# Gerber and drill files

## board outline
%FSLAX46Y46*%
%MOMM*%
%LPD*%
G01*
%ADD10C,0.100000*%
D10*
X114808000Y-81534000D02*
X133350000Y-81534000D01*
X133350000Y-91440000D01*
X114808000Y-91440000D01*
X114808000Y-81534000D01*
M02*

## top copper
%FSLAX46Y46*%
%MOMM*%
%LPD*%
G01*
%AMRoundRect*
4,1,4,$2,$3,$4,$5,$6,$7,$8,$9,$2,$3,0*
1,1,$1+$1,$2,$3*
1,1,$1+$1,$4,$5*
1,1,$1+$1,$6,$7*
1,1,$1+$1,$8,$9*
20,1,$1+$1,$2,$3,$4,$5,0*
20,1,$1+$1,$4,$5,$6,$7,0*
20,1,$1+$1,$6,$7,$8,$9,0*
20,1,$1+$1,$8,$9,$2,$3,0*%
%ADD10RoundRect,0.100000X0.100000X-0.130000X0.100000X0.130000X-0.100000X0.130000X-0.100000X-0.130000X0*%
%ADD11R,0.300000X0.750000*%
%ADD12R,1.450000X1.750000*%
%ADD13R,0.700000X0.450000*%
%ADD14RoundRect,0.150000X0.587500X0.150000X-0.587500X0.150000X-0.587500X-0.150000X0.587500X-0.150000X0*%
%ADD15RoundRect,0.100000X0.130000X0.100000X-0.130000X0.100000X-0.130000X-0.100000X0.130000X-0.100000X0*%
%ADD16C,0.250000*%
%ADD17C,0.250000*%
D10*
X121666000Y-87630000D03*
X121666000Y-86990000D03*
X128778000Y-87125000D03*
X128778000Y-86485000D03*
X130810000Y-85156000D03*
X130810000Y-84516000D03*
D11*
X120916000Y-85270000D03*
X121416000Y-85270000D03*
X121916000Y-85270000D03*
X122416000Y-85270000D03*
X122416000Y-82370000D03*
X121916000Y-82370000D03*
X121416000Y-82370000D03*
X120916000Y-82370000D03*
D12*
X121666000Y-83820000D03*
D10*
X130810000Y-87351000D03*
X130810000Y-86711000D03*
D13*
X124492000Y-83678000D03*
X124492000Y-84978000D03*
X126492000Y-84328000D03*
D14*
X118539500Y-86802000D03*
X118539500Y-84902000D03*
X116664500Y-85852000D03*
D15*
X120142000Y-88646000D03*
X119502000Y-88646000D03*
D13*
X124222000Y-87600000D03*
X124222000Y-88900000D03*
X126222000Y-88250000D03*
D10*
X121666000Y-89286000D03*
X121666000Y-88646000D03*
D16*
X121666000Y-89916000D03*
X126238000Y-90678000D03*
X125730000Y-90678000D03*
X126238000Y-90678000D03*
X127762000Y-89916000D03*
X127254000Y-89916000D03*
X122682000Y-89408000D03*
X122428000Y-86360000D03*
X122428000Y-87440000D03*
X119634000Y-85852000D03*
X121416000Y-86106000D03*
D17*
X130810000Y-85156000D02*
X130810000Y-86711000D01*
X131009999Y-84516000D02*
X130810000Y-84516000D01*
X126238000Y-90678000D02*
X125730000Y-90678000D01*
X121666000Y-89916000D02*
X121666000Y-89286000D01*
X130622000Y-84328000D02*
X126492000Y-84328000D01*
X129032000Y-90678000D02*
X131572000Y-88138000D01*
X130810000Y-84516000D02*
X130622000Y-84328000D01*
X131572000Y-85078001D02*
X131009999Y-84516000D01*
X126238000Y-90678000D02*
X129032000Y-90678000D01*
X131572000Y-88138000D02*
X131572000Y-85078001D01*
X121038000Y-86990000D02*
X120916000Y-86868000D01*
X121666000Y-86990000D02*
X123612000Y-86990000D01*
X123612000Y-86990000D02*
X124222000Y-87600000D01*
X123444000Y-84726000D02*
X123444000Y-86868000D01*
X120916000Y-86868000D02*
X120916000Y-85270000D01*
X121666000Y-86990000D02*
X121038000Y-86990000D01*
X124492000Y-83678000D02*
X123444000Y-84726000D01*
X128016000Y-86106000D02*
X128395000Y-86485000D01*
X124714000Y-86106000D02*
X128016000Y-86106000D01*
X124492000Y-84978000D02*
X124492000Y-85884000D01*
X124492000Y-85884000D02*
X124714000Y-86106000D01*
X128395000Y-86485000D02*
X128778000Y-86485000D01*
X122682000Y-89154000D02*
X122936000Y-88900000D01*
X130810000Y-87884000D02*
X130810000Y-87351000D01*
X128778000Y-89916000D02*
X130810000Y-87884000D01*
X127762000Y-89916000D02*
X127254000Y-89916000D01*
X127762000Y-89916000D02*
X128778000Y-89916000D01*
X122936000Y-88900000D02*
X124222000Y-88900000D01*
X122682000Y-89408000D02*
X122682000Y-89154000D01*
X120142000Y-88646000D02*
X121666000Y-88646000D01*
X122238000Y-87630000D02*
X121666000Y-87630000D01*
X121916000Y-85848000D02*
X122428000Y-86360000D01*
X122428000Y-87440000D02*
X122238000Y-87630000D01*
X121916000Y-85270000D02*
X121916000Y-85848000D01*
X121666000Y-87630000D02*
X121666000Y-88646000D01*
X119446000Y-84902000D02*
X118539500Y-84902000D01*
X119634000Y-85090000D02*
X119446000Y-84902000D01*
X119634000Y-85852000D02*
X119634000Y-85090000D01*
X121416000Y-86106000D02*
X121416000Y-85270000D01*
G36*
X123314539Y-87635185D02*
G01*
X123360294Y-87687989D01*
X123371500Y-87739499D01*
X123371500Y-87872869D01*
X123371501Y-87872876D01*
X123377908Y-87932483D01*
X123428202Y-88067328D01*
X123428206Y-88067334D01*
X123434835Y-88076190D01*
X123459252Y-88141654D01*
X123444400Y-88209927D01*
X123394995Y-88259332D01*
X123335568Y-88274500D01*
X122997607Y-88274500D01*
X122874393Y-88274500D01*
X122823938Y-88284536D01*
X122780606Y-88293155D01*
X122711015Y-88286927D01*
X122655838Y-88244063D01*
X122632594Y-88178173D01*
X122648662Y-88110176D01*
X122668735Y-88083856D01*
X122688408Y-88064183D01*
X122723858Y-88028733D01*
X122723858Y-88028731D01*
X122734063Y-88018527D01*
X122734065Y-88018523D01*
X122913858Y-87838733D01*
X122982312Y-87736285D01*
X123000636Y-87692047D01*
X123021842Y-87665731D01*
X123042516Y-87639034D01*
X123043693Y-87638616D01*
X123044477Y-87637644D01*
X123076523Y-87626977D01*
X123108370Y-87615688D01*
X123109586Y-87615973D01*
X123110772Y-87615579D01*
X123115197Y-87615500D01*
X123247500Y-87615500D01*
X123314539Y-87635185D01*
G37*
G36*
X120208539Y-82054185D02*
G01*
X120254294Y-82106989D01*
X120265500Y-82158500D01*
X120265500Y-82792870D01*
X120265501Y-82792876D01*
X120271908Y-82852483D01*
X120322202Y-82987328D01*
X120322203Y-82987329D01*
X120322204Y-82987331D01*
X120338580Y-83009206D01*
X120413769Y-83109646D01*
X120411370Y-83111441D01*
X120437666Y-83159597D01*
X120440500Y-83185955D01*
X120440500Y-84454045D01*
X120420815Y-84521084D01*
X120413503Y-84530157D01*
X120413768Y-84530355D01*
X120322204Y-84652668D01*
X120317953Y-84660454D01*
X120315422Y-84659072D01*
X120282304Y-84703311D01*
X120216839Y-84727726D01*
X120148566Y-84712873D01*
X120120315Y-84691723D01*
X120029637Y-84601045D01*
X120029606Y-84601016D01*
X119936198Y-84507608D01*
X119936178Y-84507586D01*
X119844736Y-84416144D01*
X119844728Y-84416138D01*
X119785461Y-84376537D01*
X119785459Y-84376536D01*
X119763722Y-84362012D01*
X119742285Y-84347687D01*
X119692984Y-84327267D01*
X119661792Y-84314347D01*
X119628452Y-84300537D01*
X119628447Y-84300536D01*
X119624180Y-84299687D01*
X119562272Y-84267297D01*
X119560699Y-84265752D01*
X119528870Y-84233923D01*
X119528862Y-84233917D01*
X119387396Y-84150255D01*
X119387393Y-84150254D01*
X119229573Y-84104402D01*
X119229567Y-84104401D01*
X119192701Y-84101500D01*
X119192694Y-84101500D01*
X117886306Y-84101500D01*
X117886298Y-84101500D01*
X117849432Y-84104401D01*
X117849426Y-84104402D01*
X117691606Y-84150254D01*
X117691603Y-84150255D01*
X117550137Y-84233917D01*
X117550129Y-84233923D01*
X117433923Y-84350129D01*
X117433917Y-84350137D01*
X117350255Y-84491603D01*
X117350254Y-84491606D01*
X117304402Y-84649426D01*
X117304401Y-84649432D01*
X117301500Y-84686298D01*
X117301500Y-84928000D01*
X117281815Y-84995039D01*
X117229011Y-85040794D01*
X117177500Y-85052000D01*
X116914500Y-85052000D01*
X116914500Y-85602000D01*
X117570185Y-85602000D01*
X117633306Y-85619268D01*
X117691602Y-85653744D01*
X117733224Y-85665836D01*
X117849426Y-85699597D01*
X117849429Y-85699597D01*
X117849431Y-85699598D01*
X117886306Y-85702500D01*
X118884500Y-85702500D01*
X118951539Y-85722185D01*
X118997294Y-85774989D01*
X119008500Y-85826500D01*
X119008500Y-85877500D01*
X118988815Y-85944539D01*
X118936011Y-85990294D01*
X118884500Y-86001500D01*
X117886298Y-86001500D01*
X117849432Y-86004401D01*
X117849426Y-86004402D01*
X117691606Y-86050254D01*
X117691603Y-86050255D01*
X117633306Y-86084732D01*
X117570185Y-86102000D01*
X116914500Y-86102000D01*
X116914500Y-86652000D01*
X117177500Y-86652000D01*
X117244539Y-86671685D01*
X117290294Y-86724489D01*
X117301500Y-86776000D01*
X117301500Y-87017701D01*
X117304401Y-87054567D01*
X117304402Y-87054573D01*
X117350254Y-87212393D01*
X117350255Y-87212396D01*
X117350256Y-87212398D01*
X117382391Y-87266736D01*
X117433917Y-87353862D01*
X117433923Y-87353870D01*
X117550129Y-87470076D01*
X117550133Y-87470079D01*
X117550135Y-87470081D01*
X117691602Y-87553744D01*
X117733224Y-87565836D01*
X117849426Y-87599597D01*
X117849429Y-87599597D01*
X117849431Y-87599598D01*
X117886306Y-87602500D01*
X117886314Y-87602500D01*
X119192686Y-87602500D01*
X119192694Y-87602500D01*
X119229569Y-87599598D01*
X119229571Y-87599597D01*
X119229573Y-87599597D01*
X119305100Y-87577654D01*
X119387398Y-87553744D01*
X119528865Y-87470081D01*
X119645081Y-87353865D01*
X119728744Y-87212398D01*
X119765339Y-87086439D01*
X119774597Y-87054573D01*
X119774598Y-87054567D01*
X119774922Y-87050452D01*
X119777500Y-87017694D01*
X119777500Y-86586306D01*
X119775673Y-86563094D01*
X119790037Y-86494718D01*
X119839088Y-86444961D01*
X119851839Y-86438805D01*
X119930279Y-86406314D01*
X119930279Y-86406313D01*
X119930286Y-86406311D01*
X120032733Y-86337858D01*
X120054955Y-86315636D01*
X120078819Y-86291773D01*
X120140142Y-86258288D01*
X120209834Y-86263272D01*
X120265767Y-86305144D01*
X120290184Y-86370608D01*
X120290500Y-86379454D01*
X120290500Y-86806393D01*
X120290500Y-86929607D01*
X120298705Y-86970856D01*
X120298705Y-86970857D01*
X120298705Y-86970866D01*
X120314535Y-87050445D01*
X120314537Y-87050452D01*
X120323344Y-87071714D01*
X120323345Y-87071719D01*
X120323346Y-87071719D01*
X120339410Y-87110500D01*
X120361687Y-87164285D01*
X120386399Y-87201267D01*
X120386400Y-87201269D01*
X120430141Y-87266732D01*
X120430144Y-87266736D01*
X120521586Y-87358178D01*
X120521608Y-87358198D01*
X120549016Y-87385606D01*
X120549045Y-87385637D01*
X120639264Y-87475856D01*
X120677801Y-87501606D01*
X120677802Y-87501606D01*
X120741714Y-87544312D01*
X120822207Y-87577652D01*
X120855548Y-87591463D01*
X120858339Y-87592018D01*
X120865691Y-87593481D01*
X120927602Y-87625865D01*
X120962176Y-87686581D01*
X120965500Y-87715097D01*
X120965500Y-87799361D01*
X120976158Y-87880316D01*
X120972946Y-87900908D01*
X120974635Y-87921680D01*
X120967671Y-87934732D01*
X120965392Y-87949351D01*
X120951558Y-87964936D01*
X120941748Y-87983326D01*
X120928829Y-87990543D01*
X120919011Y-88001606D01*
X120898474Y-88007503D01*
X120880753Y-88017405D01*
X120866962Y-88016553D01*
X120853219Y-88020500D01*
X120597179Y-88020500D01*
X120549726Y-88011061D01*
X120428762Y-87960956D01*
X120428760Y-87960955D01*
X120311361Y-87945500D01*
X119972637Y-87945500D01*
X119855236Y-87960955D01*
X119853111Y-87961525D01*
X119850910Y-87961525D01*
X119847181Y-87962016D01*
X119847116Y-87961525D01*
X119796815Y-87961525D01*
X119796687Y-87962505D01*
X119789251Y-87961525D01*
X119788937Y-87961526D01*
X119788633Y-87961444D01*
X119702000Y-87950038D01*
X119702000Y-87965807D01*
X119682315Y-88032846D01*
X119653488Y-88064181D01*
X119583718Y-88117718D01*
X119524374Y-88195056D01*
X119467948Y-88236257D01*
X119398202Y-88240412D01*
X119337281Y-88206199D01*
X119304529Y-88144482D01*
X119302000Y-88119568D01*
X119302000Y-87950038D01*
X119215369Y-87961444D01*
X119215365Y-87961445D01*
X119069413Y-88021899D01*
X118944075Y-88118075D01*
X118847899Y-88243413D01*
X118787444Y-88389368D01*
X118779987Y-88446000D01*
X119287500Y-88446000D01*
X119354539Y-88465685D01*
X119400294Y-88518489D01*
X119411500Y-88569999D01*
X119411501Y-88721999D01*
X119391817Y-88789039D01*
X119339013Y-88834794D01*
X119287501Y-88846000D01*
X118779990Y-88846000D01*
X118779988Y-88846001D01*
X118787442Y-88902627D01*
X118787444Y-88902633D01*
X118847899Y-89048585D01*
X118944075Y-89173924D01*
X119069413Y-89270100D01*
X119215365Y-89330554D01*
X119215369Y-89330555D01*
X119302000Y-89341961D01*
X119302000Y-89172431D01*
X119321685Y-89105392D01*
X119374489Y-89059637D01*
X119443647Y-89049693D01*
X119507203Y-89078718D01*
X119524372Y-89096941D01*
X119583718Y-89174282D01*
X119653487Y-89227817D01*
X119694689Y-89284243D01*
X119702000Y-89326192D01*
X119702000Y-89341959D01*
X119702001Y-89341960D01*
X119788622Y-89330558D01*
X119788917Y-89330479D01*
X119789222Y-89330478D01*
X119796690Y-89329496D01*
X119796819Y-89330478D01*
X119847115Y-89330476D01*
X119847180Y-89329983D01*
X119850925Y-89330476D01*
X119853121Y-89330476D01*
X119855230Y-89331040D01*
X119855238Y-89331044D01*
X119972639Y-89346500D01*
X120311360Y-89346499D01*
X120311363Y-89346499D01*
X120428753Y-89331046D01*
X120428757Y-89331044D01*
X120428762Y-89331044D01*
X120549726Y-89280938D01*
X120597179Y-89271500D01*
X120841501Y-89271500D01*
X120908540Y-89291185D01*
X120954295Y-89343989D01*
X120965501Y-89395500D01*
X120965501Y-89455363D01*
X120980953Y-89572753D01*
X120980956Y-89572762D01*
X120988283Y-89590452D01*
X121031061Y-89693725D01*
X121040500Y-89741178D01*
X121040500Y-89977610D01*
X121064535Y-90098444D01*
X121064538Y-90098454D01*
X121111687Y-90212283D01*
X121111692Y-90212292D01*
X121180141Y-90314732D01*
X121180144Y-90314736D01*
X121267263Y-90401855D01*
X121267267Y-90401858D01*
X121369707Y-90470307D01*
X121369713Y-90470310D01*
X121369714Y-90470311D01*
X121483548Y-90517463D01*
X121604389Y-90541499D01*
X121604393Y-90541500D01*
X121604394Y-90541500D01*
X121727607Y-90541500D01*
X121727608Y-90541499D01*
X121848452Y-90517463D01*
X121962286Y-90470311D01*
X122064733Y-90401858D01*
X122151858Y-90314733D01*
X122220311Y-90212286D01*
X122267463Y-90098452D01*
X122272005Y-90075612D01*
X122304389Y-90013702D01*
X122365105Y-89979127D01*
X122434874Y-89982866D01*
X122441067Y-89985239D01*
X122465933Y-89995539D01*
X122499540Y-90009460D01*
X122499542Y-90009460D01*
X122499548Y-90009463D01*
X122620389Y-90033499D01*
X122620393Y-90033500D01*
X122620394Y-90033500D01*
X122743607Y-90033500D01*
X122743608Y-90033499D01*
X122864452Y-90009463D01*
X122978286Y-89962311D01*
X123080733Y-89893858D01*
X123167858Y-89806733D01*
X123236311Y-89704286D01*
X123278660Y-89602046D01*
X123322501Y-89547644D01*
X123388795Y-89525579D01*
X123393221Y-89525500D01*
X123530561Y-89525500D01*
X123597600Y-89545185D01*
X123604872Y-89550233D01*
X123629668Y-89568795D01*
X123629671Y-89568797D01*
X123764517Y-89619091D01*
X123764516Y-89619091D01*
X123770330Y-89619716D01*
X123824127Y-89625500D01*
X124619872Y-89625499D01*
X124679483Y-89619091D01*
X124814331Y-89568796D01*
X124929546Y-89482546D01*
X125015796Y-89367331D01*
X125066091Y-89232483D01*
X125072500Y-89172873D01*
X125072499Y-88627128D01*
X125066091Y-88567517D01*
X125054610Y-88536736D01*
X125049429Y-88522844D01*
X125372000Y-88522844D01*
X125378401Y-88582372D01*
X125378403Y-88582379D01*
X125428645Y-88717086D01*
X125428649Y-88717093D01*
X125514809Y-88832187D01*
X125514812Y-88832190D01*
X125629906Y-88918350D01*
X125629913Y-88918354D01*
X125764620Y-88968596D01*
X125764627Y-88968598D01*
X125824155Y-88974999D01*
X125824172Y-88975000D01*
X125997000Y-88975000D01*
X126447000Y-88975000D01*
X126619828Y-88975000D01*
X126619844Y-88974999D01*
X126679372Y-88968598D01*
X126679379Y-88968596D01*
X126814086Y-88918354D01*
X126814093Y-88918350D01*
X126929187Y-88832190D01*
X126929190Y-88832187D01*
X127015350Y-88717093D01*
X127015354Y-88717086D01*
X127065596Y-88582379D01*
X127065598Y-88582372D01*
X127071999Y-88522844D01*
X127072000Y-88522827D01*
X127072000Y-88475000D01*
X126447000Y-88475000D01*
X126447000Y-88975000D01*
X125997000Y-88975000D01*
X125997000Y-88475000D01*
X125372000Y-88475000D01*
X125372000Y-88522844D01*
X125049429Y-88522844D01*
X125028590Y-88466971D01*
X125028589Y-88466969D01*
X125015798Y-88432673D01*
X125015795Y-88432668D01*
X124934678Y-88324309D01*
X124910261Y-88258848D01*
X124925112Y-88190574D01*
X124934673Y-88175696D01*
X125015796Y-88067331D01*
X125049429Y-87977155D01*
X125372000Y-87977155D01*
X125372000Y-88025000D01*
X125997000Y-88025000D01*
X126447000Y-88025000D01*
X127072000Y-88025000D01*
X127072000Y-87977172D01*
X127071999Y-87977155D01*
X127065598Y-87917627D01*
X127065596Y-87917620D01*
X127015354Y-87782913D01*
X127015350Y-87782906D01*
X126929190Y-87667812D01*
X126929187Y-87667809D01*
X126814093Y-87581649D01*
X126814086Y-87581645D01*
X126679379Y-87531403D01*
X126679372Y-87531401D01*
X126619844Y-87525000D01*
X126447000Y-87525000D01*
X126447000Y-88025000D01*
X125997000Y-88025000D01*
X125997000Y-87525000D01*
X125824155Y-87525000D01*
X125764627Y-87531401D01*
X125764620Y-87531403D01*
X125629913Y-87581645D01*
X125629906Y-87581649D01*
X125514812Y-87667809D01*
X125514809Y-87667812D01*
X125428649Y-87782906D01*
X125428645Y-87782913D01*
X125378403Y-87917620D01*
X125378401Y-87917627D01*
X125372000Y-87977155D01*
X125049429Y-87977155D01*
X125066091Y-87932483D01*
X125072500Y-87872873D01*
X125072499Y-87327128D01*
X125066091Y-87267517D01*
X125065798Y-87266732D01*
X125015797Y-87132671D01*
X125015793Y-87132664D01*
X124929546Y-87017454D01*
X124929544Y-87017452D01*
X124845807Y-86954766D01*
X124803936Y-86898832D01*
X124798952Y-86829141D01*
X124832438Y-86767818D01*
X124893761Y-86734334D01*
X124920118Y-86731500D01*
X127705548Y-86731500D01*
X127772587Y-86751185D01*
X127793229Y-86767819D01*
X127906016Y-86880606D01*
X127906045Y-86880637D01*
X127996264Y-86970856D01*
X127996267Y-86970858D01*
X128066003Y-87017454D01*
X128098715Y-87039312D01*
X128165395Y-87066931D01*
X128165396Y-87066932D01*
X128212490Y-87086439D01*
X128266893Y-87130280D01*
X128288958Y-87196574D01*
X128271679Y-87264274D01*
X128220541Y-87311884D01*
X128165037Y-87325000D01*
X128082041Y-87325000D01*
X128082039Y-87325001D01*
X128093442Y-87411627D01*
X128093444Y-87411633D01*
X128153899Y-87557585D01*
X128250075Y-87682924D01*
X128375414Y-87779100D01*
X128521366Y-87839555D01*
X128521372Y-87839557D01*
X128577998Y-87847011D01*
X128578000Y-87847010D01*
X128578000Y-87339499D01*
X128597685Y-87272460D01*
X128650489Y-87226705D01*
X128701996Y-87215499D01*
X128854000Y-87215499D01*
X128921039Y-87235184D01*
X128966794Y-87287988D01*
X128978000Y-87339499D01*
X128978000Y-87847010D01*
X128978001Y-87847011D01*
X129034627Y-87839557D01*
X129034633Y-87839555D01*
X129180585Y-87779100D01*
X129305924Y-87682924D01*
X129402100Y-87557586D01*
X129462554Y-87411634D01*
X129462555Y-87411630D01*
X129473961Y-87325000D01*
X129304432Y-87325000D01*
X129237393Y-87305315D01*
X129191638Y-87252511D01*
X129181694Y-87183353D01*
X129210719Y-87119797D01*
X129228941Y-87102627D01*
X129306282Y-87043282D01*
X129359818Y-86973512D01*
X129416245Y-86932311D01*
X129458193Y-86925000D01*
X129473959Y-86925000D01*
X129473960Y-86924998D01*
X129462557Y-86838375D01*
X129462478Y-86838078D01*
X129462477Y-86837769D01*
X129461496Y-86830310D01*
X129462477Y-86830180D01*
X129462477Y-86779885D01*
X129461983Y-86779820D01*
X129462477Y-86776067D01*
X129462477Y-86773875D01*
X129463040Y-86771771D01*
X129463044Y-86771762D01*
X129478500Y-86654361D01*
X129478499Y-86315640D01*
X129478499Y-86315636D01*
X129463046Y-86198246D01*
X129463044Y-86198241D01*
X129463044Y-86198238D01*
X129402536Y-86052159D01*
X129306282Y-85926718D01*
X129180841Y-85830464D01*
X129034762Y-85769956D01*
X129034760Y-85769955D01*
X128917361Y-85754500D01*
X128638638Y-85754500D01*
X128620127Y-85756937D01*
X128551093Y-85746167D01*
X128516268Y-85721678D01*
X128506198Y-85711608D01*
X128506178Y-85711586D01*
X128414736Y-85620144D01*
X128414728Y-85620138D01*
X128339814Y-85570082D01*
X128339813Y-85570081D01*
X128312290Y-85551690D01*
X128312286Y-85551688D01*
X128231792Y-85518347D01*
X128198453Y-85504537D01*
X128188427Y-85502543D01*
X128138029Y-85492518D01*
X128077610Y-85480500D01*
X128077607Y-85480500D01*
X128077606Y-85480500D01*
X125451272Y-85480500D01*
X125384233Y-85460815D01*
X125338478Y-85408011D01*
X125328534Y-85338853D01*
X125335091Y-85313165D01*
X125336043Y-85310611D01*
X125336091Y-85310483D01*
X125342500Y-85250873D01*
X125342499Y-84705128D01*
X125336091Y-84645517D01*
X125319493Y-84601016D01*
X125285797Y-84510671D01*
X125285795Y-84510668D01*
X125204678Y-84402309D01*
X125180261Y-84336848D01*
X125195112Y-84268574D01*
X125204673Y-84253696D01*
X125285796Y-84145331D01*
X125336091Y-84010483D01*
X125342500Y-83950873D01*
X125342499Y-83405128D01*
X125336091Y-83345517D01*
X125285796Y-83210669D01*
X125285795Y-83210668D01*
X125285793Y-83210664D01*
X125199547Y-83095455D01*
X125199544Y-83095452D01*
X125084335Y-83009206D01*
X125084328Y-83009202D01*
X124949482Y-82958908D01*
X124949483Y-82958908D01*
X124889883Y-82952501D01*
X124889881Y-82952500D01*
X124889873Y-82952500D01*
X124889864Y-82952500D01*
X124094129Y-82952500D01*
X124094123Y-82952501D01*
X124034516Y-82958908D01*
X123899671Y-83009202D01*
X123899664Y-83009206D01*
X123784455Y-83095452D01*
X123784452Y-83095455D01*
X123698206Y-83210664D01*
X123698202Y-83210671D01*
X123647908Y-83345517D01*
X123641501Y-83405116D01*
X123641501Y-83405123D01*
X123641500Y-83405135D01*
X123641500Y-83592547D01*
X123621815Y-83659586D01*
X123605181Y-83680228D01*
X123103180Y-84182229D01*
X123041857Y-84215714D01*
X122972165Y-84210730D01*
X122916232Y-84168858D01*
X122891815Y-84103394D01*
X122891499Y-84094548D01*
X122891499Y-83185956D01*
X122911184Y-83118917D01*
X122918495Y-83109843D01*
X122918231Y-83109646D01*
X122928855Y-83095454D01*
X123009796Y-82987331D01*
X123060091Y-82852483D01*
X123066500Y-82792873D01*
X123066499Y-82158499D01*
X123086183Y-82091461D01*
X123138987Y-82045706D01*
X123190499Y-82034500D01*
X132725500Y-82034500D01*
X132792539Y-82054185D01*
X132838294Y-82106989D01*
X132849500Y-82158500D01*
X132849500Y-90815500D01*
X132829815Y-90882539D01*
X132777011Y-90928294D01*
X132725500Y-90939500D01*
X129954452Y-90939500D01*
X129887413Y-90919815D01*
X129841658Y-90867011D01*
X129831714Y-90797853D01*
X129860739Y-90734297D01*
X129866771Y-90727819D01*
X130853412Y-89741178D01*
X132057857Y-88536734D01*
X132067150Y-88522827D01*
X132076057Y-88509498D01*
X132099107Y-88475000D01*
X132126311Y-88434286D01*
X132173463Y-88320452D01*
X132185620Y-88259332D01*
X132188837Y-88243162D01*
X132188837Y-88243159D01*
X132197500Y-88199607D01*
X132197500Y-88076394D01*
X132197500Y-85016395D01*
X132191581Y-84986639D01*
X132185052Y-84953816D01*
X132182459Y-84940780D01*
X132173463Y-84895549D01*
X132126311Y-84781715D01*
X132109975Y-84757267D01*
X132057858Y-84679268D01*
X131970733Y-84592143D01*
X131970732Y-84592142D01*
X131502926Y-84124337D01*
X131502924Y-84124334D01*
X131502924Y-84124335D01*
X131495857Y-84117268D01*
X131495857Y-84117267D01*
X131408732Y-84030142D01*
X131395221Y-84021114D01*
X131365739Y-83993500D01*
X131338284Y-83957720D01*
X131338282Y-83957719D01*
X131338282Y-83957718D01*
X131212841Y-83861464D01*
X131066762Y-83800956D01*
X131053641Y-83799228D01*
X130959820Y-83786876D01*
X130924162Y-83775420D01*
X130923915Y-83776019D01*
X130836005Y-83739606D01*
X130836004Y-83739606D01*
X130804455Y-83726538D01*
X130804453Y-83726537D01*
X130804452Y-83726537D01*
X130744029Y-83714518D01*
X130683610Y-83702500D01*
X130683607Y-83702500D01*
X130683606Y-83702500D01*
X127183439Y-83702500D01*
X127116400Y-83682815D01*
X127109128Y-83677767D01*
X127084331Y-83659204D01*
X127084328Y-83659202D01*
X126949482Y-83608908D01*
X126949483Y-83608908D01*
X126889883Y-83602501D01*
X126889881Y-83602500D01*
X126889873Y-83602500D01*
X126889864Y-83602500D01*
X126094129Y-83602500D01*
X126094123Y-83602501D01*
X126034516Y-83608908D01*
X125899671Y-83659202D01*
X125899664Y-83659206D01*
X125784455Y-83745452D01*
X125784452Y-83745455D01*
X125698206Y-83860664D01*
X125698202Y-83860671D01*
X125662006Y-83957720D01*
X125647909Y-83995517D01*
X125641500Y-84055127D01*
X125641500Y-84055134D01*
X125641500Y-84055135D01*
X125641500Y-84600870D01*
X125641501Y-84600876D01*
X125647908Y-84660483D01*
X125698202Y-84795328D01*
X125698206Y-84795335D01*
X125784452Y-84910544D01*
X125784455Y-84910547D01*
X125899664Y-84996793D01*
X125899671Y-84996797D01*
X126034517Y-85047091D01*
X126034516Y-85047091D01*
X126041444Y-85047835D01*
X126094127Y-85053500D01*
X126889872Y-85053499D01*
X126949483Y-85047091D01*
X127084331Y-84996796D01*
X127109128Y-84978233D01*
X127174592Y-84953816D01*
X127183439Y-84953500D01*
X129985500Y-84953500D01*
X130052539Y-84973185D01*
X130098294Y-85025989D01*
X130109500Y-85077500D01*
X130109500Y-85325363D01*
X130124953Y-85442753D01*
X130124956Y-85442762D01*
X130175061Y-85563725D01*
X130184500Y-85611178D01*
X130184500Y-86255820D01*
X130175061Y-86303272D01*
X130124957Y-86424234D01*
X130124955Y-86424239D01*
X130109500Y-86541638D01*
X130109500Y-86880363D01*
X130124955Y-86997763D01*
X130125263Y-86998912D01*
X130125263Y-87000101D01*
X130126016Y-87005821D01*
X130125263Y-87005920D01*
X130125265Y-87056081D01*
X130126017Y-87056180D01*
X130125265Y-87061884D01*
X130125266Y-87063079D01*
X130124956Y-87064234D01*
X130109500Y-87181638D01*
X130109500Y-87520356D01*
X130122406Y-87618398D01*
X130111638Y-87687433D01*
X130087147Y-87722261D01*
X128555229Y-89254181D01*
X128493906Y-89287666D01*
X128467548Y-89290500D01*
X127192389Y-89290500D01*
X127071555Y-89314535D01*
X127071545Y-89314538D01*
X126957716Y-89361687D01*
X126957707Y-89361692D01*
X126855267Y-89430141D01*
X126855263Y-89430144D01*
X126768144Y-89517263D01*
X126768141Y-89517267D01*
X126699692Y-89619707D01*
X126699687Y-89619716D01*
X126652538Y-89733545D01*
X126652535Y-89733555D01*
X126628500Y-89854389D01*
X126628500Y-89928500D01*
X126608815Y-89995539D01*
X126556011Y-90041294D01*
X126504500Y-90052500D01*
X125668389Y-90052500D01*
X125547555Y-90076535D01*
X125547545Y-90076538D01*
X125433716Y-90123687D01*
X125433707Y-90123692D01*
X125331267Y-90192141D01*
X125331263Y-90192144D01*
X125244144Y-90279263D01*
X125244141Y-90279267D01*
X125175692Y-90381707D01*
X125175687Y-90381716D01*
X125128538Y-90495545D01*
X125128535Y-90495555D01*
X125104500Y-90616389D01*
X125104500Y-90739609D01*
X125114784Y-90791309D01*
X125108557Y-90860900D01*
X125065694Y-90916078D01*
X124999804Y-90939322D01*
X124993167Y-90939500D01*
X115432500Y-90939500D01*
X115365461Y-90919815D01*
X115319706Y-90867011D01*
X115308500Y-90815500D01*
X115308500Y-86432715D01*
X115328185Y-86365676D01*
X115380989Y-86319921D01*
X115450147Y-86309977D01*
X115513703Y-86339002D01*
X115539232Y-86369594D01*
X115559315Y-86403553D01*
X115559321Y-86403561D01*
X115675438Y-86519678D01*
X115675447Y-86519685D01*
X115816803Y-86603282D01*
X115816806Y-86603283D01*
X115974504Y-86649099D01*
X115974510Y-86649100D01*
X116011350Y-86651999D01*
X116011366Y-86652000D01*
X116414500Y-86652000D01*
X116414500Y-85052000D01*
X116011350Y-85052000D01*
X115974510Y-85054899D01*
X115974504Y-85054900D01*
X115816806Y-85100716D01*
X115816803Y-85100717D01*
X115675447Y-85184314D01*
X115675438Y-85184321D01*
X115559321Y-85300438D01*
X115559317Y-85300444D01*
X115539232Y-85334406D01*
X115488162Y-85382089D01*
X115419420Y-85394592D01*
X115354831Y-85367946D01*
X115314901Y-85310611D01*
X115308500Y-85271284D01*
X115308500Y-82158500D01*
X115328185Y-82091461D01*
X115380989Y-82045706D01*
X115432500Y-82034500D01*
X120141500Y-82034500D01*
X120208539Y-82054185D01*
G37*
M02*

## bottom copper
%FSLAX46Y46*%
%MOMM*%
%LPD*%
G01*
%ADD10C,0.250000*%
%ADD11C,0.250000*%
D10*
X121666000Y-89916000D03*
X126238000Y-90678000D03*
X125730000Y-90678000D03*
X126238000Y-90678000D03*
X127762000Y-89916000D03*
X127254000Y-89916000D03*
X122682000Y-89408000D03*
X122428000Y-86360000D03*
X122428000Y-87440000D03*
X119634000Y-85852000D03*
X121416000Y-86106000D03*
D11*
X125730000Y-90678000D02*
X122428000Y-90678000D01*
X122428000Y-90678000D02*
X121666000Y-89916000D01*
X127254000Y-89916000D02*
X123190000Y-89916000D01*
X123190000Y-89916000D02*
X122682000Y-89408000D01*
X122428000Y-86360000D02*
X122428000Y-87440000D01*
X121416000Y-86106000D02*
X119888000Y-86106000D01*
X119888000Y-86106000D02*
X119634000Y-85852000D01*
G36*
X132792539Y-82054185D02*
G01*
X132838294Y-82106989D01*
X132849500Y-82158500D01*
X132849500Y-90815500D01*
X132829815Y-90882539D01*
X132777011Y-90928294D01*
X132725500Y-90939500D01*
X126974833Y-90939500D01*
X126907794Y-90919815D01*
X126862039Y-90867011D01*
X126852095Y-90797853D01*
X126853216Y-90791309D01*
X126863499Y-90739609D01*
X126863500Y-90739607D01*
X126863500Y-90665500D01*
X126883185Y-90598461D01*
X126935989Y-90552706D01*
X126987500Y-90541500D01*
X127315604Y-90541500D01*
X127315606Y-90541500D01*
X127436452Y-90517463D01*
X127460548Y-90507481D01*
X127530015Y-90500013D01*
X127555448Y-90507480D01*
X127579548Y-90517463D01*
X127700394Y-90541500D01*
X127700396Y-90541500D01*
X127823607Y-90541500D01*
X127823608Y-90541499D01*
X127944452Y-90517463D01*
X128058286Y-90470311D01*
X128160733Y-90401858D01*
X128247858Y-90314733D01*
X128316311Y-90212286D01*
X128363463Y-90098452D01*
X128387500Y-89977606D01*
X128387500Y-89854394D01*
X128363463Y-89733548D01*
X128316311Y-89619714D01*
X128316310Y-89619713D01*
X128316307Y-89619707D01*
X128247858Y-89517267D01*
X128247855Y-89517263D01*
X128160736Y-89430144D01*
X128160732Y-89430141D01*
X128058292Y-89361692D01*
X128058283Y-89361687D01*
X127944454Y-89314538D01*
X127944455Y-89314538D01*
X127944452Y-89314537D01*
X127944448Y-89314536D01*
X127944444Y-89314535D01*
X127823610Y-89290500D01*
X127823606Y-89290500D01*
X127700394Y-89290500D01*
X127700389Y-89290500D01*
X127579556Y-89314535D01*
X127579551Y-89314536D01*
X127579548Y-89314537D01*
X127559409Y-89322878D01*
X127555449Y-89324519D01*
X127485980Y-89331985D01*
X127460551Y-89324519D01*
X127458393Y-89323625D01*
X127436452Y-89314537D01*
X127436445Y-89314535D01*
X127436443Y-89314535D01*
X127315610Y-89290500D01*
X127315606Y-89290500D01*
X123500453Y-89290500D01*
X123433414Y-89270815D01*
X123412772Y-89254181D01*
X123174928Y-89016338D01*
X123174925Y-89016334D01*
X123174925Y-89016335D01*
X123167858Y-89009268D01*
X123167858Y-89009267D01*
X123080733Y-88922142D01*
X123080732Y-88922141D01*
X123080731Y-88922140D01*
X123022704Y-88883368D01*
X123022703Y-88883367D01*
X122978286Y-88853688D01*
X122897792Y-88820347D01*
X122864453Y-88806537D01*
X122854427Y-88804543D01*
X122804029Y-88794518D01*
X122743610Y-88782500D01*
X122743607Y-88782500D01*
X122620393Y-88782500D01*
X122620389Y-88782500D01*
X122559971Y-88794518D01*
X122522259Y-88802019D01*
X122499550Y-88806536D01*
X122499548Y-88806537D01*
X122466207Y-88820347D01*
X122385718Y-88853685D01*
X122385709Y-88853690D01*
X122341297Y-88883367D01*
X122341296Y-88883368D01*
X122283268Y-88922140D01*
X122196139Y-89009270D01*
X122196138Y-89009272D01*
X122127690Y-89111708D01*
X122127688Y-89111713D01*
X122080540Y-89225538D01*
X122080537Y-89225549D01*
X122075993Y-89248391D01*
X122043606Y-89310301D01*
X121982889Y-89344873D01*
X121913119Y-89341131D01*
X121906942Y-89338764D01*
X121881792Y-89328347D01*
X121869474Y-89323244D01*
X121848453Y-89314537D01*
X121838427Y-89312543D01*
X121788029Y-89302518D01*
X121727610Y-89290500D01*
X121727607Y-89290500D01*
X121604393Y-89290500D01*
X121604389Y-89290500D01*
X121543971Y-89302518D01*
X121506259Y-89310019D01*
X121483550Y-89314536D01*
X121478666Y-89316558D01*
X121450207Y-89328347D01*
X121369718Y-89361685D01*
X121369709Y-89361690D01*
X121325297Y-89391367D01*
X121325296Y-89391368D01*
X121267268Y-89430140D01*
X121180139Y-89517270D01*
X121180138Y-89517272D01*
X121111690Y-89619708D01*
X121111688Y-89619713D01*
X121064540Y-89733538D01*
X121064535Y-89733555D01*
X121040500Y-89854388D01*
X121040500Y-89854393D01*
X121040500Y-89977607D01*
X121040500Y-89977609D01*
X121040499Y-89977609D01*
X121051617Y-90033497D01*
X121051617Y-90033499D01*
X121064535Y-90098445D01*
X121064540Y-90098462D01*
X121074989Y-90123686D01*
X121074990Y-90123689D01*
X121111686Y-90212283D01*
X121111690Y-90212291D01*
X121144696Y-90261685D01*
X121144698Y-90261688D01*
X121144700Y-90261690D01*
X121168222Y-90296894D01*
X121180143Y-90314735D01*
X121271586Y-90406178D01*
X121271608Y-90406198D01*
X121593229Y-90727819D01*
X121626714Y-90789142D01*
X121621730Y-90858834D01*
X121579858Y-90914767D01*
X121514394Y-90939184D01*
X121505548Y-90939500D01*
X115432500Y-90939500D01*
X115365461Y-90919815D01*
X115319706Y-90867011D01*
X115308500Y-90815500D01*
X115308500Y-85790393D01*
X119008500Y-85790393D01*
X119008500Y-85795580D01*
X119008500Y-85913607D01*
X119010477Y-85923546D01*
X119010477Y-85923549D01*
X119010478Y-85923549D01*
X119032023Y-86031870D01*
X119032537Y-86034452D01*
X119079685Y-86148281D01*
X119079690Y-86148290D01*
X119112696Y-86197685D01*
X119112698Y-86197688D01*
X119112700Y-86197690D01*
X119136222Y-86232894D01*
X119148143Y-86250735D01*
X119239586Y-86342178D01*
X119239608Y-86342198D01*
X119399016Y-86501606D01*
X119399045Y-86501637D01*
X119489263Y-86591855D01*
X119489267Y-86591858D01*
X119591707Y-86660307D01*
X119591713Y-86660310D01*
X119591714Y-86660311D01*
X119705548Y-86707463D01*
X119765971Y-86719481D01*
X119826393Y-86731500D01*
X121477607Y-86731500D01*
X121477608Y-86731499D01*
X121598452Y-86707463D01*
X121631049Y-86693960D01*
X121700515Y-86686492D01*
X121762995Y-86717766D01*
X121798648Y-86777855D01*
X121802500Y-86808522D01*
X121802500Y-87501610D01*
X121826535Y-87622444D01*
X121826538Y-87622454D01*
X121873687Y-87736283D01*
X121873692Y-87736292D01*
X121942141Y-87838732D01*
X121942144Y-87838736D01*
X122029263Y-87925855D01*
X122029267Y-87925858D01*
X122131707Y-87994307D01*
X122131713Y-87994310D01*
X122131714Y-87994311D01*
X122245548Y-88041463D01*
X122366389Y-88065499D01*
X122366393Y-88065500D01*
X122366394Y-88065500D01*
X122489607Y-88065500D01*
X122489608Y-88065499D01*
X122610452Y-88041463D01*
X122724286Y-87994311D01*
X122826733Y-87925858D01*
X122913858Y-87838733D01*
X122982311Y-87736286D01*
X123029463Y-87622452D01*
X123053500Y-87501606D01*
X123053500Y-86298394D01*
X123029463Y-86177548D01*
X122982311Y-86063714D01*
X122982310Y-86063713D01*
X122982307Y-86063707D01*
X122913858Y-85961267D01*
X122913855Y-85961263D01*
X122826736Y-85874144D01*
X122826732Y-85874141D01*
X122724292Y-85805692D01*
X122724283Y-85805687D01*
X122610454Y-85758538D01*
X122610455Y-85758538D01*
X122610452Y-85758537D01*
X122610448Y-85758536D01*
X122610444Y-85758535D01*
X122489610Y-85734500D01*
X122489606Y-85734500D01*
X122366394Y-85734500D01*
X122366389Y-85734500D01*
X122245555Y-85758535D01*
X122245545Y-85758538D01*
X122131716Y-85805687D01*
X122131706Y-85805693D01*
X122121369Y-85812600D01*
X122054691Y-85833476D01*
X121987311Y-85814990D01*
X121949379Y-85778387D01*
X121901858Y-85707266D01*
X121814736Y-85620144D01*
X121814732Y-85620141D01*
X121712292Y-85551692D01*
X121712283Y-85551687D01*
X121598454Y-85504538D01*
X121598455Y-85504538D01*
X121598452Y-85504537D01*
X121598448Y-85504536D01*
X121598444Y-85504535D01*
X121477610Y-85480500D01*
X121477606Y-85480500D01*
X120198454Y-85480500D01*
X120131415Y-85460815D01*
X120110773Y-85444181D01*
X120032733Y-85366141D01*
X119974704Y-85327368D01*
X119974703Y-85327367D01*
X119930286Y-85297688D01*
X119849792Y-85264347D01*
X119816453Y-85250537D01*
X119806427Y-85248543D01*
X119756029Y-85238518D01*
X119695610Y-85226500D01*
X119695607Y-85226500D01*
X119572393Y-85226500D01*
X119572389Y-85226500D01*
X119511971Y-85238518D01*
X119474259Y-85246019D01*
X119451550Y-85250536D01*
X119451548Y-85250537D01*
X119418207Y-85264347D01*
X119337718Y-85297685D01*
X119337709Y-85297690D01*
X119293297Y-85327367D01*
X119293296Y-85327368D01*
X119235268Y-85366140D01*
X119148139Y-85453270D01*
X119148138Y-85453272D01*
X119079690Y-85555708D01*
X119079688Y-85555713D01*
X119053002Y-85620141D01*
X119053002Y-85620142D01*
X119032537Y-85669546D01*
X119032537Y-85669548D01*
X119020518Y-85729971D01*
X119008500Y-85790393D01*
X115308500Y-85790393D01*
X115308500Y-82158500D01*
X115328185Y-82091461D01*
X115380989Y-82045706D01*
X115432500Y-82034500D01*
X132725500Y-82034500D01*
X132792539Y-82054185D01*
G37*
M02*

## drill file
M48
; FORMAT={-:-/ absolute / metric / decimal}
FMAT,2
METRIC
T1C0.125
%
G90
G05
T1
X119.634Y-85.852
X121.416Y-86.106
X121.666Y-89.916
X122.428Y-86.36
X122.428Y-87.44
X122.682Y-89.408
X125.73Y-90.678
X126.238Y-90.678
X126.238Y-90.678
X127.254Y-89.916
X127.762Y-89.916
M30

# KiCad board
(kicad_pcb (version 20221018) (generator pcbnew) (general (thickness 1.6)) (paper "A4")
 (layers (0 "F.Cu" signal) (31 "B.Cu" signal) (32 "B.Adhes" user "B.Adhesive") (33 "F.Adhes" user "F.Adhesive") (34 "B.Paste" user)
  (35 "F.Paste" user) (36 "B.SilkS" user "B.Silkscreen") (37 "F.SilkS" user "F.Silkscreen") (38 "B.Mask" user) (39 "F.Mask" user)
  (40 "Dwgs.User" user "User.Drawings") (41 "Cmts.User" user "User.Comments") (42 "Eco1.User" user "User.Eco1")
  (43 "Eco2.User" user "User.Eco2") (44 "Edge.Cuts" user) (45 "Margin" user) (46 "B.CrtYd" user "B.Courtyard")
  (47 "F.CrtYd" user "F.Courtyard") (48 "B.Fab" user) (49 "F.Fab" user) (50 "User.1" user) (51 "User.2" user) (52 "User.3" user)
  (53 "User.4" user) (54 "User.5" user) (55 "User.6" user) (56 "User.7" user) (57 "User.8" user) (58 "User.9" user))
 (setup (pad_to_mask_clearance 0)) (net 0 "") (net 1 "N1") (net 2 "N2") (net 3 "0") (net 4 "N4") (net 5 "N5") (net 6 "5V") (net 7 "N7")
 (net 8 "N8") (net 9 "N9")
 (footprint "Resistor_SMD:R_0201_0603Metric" (layer "F.Cu") (at 121.666 87.31 90)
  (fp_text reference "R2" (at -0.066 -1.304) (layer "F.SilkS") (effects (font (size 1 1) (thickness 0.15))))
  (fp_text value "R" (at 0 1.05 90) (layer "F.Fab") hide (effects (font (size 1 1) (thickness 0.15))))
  (pad "" smd roundrect (at -0.345 0 90) (size 0.318 0.36) (layers "F.Paste") (roundrect_rratio 0.25))
  (pad "" smd roundrect (at 0.345 0 90) (size 0.318 0.36) (layers "F.Paste") (roundrect_rratio 0.25))
  (pad "1" smd roundrect (at -0.32 0 90) (size 0.46 0.4) (layers "F.Cu" "F.Mask") (roundrect_rratio 0.25) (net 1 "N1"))
  (pad "2" smd roundrect (at 0.32 0 90) (size 0.46 0.4) (layers "F.Cu" "F.Mask") (roundrect_rratio 0.25) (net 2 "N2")))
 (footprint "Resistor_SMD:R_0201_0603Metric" (layer "F.Cu") (at 128.778 86.805 90)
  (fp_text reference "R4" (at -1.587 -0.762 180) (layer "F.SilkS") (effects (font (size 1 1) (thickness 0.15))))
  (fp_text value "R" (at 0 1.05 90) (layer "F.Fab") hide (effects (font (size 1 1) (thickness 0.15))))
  (pad "" smd roundrect (at -0.345 0 90) (size 0.318 0.36) (layers "F.Paste") (roundrect_rratio 0.25))
  (pad "" smd roundrect (at 0.345 0 90) (size 0.318 0.36) (layers "F.Paste") (roundrect_rratio 0.25))
  (pad "1" smd roundrect (at -0.32 0 90) (size 0.46 0.4) (layers "F.Cu" "F.Mask") (roundrect_rratio 0.25) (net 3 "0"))
  (pad "2" smd roundrect (at 0.32 0 90) (size 0.46 0.4) (layers "F.Cu" "F.Mask") (roundrect_rratio 0.25) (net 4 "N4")))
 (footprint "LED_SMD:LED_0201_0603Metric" (layer "F.Cu") (at 130.81 84.836 90)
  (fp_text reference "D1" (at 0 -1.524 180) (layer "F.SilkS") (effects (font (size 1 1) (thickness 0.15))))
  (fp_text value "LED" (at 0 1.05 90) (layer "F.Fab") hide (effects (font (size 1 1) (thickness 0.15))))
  (pad "" smd roundrect (at -0.345 0 90) (size 0.318 0.36) (layers "F.Paste") (roundrect_rratio 0.25))
  (pad "" smd roundrect (at 0.345 0 90) (size 0.318 0.36) (layers "F.Paste") (roundrect_rratio 0.25))
  (pad "1" smd roundrect (at -0.32 0 90) (size 0.46 0.4) (layers "F.Cu" "F.Mask") (roundrect_rratio 0.25) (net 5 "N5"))
  (pad "2" smd roundrect (at 0.32 0 90) (size 0.46 0.4) (layers "F.Cu" "F.Mask") (roundrect_rratio 0.25) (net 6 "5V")))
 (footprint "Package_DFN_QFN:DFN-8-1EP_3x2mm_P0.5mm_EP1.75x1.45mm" (layer "F.Cu") (at 121.666 83.82 90)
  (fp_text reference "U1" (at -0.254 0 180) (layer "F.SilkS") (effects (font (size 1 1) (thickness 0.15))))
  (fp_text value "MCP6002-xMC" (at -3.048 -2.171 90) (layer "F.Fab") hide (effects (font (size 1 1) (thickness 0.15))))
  (pad "" smd rect (at -0.4375 -0.3625 90) (size 0.71 0.58) (layers "F.Paste"))
  (pad "" smd rect (at -0.4375 0.3625 90) (size 0.71 0.58) (layers "F.Paste"))
  (pad "" smd rect (at 0.4375 -0.3625 90) (size 0.71 0.58) (layers "F.Paste"))
  (pad "" smd rect (at 0.4375 0.3625 90) (size 0.71 0.58) (layers "F.Paste"))
  (pad "1" smd rect (at -1.45 -0.75 90) (size 0.75 0.3) (layers "F.Cu" "F.Paste" "F.Mask") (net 2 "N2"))
  (pad "2" smd rect (at -1.45 -0.25 90) (size 0.75 0.3) (layers "F.Cu" "F.Paste" "F.Mask") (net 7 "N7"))
  (pad "3" smd rect (at -1.45 0.25 90) (size 0.75 0.3) (layers "F.Cu" "F.Paste" "F.Mask") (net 1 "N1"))
  (pad "4" smd rect (at -1.45 0.75 90) (size 0.75 0.3) (layers "F.Cu" "F.Paste" "F.Mask"))
  (pad "5" smd rect (at 1.45 0.75 90) (size 0.75 0.3) (layers "F.Cu" "F.Paste" "F.Mask"))
  (pad "6" smd rect (at 1.45 0.25 90) (size 0.75 0.3) (layers "F.Cu" "F.Paste" "F.Mask"))
  (pad "7" smd rect (at 1.45 -0.25 90) (size 0.75 0.3) (layers "F.Cu" "F.Paste" "F.Mask"))
  (pad "8" smd rect (at 1.45 -0.75 90) (size 0.75 0.3) (layers "F.Cu" "F.Paste" "F.Mask"))
  (pad "9" smd rect (at 0 0 90) (size 1.75 1.45) (layers "F.Cu" "F.Mask")))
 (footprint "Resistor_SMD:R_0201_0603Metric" (layer "F.Cu") (at 130.81 87.031 90)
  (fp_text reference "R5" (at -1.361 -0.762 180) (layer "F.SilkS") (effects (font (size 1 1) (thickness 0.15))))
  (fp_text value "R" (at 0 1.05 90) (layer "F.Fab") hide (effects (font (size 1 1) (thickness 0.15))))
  (pad "" smd roundrect (at -0.345 0 90) (size 0.318 0.36) (layers "F.Paste") (roundrect_rratio 0.25))
  (pad "" smd roundrect (at 0.345 0 90) (size 0.318 0.36) (layers "F.Paste") (roundrect_rratio 0.25))
  (pad "1" smd roundrect (at -0.32 0 90) (size 0.46 0.4) (layers "F.Cu" "F.Mask") (roundrect_rratio 0.25) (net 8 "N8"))
  (pad "2" smd roundrect (at 0.32 0 90) (size 0.46 0.4) (layers "F.Cu" "F.Mask") (roundrect_rratio 0.25) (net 5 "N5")))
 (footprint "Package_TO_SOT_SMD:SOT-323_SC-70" (layer "F.Cu") (at 125.492 84.328)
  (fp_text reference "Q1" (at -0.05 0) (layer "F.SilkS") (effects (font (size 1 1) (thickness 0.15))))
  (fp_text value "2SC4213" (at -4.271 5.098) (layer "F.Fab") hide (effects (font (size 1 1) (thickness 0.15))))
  (pad "1" smd rect (at -1 -0.65 270) (size 0.45 0.7) (layers "F.Cu" "F.Paste" "F.Mask") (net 2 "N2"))
  (pad "2" smd rect (at -1 0.65 270) (size 0.45 0.7) (layers "F.Cu" "F.Paste" "F.Mask") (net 4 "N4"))
  (pad "3" smd rect (at 1 0 270) (size 0.45 0.7) (layers "F.Cu" "F.Paste" "F.Mask") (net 6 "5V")))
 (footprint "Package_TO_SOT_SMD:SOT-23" (layer "F.Cu") (at 117.602 85.852 180)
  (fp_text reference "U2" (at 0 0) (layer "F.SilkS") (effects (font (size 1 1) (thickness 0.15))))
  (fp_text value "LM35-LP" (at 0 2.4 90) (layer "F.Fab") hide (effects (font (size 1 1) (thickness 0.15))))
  (pad "1" smd roundrect (at -0.9375 -0.95 180) (size 1.475 0.6) (layers "F.Cu" "F.Paste" "F.Mask") (roundrect_rratio 0.25) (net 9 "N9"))
  (pad "2" smd roundrect (at -0.9375 0.95 180) (size 1.475 0.6) (layers "F.Cu" "F.Paste" "F.Mask") (roundrect_rratio 0.25) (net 7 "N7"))
  (pad "3" smd roundrect (at 0.9375 0 180) (size 1.475 0.6) (layers "F.Cu" "F.Paste" "F.Mask") (roundrect_rratio 0.25) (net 3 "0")))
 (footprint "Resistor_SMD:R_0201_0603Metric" (layer "F.Cu") (at 119.822 88.646 180)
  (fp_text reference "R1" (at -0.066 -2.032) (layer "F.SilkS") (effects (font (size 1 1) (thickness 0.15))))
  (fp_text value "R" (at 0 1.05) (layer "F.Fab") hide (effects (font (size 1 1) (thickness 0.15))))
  (pad "" smd roundrect (at -0.345 0 180) (size 0.318 0.36) (layers "F.Paste") (roundrect_rratio 0.25))
  (pad "" smd roundrect (at 0.345 0 180) (size 0.318 0.36) (layers "F.Paste") (roundrect_rratio 0.25))
  (pad "1" smd roundrect (at -0.32 0 180) (size 0.46 0.4) (layers "F.Cu" "F.Mask") (roundrect_rratio 0.25) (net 1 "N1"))
  (pad "2" smd roundrect (at 0.32 0 180) (size 0.46 0.4) (layers "F.Cu" "F.Mask") (roundrect_rratio 0.25) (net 3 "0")))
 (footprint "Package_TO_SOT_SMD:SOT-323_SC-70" (layer "F.Cu") (at 125.222 88.25)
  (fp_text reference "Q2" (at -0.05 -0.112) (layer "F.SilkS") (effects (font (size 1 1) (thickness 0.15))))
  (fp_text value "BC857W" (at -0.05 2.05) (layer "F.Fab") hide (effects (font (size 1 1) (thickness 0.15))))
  (pad "1" smd rect (at -1 -0.65 270) (size 0.45 0.7) (layers "F.Cu" "F.Paste" "F.Mask") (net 2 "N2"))
  (pad "2" smd rect (at -1 0.65 270) (size 0.45 0.7) (layers "F.Cu" "F.Paste" "F.Mask") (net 8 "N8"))
  (pad "3" smd rect (at 1 0 270) (size 0.45 0.7) (layers "F.Cu" "F.Paste" "F.Mask") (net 3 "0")))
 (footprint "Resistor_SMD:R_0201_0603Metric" (layer "F.Cu") (at 121.666 88.966 90)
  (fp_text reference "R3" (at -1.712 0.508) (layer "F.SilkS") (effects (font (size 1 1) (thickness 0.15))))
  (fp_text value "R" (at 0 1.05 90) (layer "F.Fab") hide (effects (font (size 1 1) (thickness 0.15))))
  (pad "" smd roundrect (at -0.345 0 90) (size 0.318 0.36) (layers "F.Paste") (roundrect_rratio 0.25))
  (pad "" smd roundrect (at 0.345 0 90) (size 0.318 0.36) (layers "F.Paste") (roundrect_rratio 0.25))
  (pad "1" smd roundrect (at -0.32 0 90) (size 0.46 0.4) (layers "F.Cu" "F.Mask") (roundrect_rratio 0.25) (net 6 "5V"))
  (pad "2" smd roundrect (at 0.32 0 90) (size 0.46 0.4) (layers "F.Cu" "F.Mask") (roundrect_rratio 0.25) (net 1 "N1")))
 (gr_rect (start 114.808 81.534) (end 133.35 91.44) (stroke (width 0.1) (type default)) (fill none) (layer "Edge.Cuts"))
 (segment (start 130.81 85.156) (end 130.81 86.711) (width 0.25) (layer "F.Cu") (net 5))
 (segment (start 131.009999 84.516) (end 130.81 84.516) (width 0.25) (layer "F.Cu") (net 6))
 (segment (start 126.238 90.678) (end 125.73 90.678) (width 0.25) (layer "F.Cu") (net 6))
 (segment (start 121.666 89.916) (end 121.666 89.286) (width 0.25) (layer "F.Cu") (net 6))
 (segment (start 130.622 84.328) (end 126.492 84.328) (width 0.25) (layer "F.Cu") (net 6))
 (segment (start 129.032 90.678) (end 131.572 88.138) (width 0.25) (layer "F.Cu") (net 6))
 (segment (start 130.81 84.516) (end 130.622 84.328) (width 0.25) (layer "F.Cu") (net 6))
 (segment (start 131.572 85.078001) (end 131.009999 84.516) (width 0.25) (layer "F.Cu") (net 6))
 (segment (start 126.238 90.678) (end 129.032 90.678) (width 0.25) (layer "F.Cu") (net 6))
 (segment (start 131.572 88.138) (end 131.572 85.078001) (width 0.25) (layer "F.Cu") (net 6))
 (via (at 121.666 89.916) (size 0.25) (drill 0.125) (layers "F.Cu" "B.Cu") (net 6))
 (via (at 126.238 90.678) (size 0.25) (drill 0.125) (layers "F.Cu" "B.Cu") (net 6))
 (via (at 125.73 90.678) (size 0.25) (drill 0.125) (layers "F.Cu" "B.Cu") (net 6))
 (via (at 126.238 90.678) (size 0.25) (drill 0.125) (layers "F.Cu" "B.Cu") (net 6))
 (segment (start 125.73 90.678) (end 122.428 90.678) (width 0.25) (layer "B.Cu") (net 6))
 (segment (start 122.428 90.678) (end 121.666 89.916) (width 0.25) (layer "B.Cu") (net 6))
 (segment (start 121.038 86.99) (end 120.916 86.868) (width 0.25) (layer "F.Cu") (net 2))
 (segment (start 121.666 86.99) (end 123.612 86.99) (width 0.25) (layer "F.Cu") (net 2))
 (segment (start 123.612 86.99) (end 124.222 87.6) (width 0.25) (layer "F.Cu") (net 2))
 (segment (start 123.444 84.726) (end 123.444 86.868) (width 0.25) (layer "F.Cu") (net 2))
 (segment (start 120.916 86.868) (end 120.916 85.27) (width 0.25) (layer "F.Cu") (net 2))
 (segment (start 121.666 86.99) (end 121.038 86.99) (width 0.25) (layer "F.Cu") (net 2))
 (segment (start 124.492 83.678) (end 123.444 84.726) (width 0.25) (layer "F.Cu") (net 2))
 (segment (start 128.016 86.106) (end 128.395 86.485) (width 0.25) (layer "F.Cu") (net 4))
 (segment (start 124.714 86.106) (end 128.016 86.106) (width 0.25) (layer "F.Cu") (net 4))
 (segment (start 124.492 84.978) (end 124.492 85.884) (width 0.25) (layer "F.Cu") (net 4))
 (segment (start 124.492 85.884) (end 124.714 86.106) (width 0.25) (layer "F.Cu") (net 4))
 (segment (start 128.395 86.485) (end 128.778 86.485) (width 0.25) (layer "F.Cu") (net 4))
 (segment (start 122.682 89.154) (end 122.936 88.9) (width 0.25) (layer "F.Cu") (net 8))
 (segment (start 130.81 87.884) (end 130.81 87.351) (width 0.25) (layer "F.Cu") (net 8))
 (segment (start 128.778 89.916) (end 130.81 87.884) (width 0.25) (layer "F.Cu") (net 8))
 (segment (start 127.762 89.916) (end 127.254 89.916) (width 0.25) (layer "F.Cu") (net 8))
 (segment (start 127.762 89.916) (end 128.778 89.916) (width 0.25) (layer "F.Cu") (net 8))
 (segment (start 122.936 88.9) (end 124.222 88.9) (width 0.25) (layer "F.Cu") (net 8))
 (segment (start 122.682 89.408) (end 122.682 89.154) (width 0.25) (layer "F.Cu") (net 8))
 (via (at 127.762 89.916) (size 0.25) (drill 0.125) (layers "F.Cu" "B.Cu") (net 8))
 (via (at 127.254 89.916) (size 0.25) (drill 0.125) (layers "F.Cu" "B.Cu") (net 8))
 (via (at 122.682 89.408) (size 0.25) (drill 0.125) (layers "F.Cu" "B.Cu") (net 8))
 (segment (start 127.254 89.916) (end 123.19 89.916) (width 0.25) (layer "B.Cu") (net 8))
 (segment (start 123.19 89.916) (end 122.682 89.408) (width 0.25) (layer "B.Cu") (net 8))
 (segment (start 120.142 88.646) (end 121.666 88.646) (width 0.25) (layer "F.Cu") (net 1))
 (segment (start 122.238 87.63) (end 121.666 87.63) (width 0.25) (layer "F.Cu") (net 1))
 (segment (start 121.916 85.848) (end 122.428 86.36) (width 0.25) (layer "F.Cu") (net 1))
 (segment (start 122.428 87.44) (end 122.238 87.63) (width 0.25) (layer "F.Cu") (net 1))
 (segment (start 121.916 85.27) (end 121.916 85.848) (width 0.25) (layer "F.Cu") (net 1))
 (segment (start 121.666 87.63) (end 121.666 88.646) (width 0.25) (layer "F.Cu") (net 1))
 (via (at 122.428 86.36) (size 0.25) (drill 0.125) (layers "F.Cu" "B.Cu") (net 1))
 (via (at 122.428 87.44) (size 0.25) (drill 0.125) (layers "F.Cu" "B.Cu") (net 1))
 (segment (start 122.428 86.36) (end 122.428 87.44) (width 0.25) (layer "B.Cu") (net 1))
 (segment (start 119.446 84.902) (end 118.5395 84.902) (width 0.25) (layer "F.Cu") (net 7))
 (segment (start 119.634 85.09) (end 119.446 84.902) (width 0.25) (layer "F.Cu") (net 7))
 (segment (start 119.634 85.852) (end 119.634 85.09) (width 0.25) (layer "F.Cu") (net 7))
 (segment (start 121.416 86.106) (end 121.416 85.27) (width 0.25) (layer "F.Cu") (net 7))
 (via (at 119.634 85.852) (size 0.25) (drill 0.125) (layers "F.Cu" "B.Cu") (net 7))
 (via (at 121.416 86.106) (size 0.25) (drill 0.125) (layers "F.Cu" "B.Cu") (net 7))
 (segment (start 121.416 86.106) (end 119.888 86.106) (width 0.25) (layer "B.Cu") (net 7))
 (segment (start 119.888 86.106) (end 119.634 85.852) (width 0.25) (layer "B.Cu") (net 7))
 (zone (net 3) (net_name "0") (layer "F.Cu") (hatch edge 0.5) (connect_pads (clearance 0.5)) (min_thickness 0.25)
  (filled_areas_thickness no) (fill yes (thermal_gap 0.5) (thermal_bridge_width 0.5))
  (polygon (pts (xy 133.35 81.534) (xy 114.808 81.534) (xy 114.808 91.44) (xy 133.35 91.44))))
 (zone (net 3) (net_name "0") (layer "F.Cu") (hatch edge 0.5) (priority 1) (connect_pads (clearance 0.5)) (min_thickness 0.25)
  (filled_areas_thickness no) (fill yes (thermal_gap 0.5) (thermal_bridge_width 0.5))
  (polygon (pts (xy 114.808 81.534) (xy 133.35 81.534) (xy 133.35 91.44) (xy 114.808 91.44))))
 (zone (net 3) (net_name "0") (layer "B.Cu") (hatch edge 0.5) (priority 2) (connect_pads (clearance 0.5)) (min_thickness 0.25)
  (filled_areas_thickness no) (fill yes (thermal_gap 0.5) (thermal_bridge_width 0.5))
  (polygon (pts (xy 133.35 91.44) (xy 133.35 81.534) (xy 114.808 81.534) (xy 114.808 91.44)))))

